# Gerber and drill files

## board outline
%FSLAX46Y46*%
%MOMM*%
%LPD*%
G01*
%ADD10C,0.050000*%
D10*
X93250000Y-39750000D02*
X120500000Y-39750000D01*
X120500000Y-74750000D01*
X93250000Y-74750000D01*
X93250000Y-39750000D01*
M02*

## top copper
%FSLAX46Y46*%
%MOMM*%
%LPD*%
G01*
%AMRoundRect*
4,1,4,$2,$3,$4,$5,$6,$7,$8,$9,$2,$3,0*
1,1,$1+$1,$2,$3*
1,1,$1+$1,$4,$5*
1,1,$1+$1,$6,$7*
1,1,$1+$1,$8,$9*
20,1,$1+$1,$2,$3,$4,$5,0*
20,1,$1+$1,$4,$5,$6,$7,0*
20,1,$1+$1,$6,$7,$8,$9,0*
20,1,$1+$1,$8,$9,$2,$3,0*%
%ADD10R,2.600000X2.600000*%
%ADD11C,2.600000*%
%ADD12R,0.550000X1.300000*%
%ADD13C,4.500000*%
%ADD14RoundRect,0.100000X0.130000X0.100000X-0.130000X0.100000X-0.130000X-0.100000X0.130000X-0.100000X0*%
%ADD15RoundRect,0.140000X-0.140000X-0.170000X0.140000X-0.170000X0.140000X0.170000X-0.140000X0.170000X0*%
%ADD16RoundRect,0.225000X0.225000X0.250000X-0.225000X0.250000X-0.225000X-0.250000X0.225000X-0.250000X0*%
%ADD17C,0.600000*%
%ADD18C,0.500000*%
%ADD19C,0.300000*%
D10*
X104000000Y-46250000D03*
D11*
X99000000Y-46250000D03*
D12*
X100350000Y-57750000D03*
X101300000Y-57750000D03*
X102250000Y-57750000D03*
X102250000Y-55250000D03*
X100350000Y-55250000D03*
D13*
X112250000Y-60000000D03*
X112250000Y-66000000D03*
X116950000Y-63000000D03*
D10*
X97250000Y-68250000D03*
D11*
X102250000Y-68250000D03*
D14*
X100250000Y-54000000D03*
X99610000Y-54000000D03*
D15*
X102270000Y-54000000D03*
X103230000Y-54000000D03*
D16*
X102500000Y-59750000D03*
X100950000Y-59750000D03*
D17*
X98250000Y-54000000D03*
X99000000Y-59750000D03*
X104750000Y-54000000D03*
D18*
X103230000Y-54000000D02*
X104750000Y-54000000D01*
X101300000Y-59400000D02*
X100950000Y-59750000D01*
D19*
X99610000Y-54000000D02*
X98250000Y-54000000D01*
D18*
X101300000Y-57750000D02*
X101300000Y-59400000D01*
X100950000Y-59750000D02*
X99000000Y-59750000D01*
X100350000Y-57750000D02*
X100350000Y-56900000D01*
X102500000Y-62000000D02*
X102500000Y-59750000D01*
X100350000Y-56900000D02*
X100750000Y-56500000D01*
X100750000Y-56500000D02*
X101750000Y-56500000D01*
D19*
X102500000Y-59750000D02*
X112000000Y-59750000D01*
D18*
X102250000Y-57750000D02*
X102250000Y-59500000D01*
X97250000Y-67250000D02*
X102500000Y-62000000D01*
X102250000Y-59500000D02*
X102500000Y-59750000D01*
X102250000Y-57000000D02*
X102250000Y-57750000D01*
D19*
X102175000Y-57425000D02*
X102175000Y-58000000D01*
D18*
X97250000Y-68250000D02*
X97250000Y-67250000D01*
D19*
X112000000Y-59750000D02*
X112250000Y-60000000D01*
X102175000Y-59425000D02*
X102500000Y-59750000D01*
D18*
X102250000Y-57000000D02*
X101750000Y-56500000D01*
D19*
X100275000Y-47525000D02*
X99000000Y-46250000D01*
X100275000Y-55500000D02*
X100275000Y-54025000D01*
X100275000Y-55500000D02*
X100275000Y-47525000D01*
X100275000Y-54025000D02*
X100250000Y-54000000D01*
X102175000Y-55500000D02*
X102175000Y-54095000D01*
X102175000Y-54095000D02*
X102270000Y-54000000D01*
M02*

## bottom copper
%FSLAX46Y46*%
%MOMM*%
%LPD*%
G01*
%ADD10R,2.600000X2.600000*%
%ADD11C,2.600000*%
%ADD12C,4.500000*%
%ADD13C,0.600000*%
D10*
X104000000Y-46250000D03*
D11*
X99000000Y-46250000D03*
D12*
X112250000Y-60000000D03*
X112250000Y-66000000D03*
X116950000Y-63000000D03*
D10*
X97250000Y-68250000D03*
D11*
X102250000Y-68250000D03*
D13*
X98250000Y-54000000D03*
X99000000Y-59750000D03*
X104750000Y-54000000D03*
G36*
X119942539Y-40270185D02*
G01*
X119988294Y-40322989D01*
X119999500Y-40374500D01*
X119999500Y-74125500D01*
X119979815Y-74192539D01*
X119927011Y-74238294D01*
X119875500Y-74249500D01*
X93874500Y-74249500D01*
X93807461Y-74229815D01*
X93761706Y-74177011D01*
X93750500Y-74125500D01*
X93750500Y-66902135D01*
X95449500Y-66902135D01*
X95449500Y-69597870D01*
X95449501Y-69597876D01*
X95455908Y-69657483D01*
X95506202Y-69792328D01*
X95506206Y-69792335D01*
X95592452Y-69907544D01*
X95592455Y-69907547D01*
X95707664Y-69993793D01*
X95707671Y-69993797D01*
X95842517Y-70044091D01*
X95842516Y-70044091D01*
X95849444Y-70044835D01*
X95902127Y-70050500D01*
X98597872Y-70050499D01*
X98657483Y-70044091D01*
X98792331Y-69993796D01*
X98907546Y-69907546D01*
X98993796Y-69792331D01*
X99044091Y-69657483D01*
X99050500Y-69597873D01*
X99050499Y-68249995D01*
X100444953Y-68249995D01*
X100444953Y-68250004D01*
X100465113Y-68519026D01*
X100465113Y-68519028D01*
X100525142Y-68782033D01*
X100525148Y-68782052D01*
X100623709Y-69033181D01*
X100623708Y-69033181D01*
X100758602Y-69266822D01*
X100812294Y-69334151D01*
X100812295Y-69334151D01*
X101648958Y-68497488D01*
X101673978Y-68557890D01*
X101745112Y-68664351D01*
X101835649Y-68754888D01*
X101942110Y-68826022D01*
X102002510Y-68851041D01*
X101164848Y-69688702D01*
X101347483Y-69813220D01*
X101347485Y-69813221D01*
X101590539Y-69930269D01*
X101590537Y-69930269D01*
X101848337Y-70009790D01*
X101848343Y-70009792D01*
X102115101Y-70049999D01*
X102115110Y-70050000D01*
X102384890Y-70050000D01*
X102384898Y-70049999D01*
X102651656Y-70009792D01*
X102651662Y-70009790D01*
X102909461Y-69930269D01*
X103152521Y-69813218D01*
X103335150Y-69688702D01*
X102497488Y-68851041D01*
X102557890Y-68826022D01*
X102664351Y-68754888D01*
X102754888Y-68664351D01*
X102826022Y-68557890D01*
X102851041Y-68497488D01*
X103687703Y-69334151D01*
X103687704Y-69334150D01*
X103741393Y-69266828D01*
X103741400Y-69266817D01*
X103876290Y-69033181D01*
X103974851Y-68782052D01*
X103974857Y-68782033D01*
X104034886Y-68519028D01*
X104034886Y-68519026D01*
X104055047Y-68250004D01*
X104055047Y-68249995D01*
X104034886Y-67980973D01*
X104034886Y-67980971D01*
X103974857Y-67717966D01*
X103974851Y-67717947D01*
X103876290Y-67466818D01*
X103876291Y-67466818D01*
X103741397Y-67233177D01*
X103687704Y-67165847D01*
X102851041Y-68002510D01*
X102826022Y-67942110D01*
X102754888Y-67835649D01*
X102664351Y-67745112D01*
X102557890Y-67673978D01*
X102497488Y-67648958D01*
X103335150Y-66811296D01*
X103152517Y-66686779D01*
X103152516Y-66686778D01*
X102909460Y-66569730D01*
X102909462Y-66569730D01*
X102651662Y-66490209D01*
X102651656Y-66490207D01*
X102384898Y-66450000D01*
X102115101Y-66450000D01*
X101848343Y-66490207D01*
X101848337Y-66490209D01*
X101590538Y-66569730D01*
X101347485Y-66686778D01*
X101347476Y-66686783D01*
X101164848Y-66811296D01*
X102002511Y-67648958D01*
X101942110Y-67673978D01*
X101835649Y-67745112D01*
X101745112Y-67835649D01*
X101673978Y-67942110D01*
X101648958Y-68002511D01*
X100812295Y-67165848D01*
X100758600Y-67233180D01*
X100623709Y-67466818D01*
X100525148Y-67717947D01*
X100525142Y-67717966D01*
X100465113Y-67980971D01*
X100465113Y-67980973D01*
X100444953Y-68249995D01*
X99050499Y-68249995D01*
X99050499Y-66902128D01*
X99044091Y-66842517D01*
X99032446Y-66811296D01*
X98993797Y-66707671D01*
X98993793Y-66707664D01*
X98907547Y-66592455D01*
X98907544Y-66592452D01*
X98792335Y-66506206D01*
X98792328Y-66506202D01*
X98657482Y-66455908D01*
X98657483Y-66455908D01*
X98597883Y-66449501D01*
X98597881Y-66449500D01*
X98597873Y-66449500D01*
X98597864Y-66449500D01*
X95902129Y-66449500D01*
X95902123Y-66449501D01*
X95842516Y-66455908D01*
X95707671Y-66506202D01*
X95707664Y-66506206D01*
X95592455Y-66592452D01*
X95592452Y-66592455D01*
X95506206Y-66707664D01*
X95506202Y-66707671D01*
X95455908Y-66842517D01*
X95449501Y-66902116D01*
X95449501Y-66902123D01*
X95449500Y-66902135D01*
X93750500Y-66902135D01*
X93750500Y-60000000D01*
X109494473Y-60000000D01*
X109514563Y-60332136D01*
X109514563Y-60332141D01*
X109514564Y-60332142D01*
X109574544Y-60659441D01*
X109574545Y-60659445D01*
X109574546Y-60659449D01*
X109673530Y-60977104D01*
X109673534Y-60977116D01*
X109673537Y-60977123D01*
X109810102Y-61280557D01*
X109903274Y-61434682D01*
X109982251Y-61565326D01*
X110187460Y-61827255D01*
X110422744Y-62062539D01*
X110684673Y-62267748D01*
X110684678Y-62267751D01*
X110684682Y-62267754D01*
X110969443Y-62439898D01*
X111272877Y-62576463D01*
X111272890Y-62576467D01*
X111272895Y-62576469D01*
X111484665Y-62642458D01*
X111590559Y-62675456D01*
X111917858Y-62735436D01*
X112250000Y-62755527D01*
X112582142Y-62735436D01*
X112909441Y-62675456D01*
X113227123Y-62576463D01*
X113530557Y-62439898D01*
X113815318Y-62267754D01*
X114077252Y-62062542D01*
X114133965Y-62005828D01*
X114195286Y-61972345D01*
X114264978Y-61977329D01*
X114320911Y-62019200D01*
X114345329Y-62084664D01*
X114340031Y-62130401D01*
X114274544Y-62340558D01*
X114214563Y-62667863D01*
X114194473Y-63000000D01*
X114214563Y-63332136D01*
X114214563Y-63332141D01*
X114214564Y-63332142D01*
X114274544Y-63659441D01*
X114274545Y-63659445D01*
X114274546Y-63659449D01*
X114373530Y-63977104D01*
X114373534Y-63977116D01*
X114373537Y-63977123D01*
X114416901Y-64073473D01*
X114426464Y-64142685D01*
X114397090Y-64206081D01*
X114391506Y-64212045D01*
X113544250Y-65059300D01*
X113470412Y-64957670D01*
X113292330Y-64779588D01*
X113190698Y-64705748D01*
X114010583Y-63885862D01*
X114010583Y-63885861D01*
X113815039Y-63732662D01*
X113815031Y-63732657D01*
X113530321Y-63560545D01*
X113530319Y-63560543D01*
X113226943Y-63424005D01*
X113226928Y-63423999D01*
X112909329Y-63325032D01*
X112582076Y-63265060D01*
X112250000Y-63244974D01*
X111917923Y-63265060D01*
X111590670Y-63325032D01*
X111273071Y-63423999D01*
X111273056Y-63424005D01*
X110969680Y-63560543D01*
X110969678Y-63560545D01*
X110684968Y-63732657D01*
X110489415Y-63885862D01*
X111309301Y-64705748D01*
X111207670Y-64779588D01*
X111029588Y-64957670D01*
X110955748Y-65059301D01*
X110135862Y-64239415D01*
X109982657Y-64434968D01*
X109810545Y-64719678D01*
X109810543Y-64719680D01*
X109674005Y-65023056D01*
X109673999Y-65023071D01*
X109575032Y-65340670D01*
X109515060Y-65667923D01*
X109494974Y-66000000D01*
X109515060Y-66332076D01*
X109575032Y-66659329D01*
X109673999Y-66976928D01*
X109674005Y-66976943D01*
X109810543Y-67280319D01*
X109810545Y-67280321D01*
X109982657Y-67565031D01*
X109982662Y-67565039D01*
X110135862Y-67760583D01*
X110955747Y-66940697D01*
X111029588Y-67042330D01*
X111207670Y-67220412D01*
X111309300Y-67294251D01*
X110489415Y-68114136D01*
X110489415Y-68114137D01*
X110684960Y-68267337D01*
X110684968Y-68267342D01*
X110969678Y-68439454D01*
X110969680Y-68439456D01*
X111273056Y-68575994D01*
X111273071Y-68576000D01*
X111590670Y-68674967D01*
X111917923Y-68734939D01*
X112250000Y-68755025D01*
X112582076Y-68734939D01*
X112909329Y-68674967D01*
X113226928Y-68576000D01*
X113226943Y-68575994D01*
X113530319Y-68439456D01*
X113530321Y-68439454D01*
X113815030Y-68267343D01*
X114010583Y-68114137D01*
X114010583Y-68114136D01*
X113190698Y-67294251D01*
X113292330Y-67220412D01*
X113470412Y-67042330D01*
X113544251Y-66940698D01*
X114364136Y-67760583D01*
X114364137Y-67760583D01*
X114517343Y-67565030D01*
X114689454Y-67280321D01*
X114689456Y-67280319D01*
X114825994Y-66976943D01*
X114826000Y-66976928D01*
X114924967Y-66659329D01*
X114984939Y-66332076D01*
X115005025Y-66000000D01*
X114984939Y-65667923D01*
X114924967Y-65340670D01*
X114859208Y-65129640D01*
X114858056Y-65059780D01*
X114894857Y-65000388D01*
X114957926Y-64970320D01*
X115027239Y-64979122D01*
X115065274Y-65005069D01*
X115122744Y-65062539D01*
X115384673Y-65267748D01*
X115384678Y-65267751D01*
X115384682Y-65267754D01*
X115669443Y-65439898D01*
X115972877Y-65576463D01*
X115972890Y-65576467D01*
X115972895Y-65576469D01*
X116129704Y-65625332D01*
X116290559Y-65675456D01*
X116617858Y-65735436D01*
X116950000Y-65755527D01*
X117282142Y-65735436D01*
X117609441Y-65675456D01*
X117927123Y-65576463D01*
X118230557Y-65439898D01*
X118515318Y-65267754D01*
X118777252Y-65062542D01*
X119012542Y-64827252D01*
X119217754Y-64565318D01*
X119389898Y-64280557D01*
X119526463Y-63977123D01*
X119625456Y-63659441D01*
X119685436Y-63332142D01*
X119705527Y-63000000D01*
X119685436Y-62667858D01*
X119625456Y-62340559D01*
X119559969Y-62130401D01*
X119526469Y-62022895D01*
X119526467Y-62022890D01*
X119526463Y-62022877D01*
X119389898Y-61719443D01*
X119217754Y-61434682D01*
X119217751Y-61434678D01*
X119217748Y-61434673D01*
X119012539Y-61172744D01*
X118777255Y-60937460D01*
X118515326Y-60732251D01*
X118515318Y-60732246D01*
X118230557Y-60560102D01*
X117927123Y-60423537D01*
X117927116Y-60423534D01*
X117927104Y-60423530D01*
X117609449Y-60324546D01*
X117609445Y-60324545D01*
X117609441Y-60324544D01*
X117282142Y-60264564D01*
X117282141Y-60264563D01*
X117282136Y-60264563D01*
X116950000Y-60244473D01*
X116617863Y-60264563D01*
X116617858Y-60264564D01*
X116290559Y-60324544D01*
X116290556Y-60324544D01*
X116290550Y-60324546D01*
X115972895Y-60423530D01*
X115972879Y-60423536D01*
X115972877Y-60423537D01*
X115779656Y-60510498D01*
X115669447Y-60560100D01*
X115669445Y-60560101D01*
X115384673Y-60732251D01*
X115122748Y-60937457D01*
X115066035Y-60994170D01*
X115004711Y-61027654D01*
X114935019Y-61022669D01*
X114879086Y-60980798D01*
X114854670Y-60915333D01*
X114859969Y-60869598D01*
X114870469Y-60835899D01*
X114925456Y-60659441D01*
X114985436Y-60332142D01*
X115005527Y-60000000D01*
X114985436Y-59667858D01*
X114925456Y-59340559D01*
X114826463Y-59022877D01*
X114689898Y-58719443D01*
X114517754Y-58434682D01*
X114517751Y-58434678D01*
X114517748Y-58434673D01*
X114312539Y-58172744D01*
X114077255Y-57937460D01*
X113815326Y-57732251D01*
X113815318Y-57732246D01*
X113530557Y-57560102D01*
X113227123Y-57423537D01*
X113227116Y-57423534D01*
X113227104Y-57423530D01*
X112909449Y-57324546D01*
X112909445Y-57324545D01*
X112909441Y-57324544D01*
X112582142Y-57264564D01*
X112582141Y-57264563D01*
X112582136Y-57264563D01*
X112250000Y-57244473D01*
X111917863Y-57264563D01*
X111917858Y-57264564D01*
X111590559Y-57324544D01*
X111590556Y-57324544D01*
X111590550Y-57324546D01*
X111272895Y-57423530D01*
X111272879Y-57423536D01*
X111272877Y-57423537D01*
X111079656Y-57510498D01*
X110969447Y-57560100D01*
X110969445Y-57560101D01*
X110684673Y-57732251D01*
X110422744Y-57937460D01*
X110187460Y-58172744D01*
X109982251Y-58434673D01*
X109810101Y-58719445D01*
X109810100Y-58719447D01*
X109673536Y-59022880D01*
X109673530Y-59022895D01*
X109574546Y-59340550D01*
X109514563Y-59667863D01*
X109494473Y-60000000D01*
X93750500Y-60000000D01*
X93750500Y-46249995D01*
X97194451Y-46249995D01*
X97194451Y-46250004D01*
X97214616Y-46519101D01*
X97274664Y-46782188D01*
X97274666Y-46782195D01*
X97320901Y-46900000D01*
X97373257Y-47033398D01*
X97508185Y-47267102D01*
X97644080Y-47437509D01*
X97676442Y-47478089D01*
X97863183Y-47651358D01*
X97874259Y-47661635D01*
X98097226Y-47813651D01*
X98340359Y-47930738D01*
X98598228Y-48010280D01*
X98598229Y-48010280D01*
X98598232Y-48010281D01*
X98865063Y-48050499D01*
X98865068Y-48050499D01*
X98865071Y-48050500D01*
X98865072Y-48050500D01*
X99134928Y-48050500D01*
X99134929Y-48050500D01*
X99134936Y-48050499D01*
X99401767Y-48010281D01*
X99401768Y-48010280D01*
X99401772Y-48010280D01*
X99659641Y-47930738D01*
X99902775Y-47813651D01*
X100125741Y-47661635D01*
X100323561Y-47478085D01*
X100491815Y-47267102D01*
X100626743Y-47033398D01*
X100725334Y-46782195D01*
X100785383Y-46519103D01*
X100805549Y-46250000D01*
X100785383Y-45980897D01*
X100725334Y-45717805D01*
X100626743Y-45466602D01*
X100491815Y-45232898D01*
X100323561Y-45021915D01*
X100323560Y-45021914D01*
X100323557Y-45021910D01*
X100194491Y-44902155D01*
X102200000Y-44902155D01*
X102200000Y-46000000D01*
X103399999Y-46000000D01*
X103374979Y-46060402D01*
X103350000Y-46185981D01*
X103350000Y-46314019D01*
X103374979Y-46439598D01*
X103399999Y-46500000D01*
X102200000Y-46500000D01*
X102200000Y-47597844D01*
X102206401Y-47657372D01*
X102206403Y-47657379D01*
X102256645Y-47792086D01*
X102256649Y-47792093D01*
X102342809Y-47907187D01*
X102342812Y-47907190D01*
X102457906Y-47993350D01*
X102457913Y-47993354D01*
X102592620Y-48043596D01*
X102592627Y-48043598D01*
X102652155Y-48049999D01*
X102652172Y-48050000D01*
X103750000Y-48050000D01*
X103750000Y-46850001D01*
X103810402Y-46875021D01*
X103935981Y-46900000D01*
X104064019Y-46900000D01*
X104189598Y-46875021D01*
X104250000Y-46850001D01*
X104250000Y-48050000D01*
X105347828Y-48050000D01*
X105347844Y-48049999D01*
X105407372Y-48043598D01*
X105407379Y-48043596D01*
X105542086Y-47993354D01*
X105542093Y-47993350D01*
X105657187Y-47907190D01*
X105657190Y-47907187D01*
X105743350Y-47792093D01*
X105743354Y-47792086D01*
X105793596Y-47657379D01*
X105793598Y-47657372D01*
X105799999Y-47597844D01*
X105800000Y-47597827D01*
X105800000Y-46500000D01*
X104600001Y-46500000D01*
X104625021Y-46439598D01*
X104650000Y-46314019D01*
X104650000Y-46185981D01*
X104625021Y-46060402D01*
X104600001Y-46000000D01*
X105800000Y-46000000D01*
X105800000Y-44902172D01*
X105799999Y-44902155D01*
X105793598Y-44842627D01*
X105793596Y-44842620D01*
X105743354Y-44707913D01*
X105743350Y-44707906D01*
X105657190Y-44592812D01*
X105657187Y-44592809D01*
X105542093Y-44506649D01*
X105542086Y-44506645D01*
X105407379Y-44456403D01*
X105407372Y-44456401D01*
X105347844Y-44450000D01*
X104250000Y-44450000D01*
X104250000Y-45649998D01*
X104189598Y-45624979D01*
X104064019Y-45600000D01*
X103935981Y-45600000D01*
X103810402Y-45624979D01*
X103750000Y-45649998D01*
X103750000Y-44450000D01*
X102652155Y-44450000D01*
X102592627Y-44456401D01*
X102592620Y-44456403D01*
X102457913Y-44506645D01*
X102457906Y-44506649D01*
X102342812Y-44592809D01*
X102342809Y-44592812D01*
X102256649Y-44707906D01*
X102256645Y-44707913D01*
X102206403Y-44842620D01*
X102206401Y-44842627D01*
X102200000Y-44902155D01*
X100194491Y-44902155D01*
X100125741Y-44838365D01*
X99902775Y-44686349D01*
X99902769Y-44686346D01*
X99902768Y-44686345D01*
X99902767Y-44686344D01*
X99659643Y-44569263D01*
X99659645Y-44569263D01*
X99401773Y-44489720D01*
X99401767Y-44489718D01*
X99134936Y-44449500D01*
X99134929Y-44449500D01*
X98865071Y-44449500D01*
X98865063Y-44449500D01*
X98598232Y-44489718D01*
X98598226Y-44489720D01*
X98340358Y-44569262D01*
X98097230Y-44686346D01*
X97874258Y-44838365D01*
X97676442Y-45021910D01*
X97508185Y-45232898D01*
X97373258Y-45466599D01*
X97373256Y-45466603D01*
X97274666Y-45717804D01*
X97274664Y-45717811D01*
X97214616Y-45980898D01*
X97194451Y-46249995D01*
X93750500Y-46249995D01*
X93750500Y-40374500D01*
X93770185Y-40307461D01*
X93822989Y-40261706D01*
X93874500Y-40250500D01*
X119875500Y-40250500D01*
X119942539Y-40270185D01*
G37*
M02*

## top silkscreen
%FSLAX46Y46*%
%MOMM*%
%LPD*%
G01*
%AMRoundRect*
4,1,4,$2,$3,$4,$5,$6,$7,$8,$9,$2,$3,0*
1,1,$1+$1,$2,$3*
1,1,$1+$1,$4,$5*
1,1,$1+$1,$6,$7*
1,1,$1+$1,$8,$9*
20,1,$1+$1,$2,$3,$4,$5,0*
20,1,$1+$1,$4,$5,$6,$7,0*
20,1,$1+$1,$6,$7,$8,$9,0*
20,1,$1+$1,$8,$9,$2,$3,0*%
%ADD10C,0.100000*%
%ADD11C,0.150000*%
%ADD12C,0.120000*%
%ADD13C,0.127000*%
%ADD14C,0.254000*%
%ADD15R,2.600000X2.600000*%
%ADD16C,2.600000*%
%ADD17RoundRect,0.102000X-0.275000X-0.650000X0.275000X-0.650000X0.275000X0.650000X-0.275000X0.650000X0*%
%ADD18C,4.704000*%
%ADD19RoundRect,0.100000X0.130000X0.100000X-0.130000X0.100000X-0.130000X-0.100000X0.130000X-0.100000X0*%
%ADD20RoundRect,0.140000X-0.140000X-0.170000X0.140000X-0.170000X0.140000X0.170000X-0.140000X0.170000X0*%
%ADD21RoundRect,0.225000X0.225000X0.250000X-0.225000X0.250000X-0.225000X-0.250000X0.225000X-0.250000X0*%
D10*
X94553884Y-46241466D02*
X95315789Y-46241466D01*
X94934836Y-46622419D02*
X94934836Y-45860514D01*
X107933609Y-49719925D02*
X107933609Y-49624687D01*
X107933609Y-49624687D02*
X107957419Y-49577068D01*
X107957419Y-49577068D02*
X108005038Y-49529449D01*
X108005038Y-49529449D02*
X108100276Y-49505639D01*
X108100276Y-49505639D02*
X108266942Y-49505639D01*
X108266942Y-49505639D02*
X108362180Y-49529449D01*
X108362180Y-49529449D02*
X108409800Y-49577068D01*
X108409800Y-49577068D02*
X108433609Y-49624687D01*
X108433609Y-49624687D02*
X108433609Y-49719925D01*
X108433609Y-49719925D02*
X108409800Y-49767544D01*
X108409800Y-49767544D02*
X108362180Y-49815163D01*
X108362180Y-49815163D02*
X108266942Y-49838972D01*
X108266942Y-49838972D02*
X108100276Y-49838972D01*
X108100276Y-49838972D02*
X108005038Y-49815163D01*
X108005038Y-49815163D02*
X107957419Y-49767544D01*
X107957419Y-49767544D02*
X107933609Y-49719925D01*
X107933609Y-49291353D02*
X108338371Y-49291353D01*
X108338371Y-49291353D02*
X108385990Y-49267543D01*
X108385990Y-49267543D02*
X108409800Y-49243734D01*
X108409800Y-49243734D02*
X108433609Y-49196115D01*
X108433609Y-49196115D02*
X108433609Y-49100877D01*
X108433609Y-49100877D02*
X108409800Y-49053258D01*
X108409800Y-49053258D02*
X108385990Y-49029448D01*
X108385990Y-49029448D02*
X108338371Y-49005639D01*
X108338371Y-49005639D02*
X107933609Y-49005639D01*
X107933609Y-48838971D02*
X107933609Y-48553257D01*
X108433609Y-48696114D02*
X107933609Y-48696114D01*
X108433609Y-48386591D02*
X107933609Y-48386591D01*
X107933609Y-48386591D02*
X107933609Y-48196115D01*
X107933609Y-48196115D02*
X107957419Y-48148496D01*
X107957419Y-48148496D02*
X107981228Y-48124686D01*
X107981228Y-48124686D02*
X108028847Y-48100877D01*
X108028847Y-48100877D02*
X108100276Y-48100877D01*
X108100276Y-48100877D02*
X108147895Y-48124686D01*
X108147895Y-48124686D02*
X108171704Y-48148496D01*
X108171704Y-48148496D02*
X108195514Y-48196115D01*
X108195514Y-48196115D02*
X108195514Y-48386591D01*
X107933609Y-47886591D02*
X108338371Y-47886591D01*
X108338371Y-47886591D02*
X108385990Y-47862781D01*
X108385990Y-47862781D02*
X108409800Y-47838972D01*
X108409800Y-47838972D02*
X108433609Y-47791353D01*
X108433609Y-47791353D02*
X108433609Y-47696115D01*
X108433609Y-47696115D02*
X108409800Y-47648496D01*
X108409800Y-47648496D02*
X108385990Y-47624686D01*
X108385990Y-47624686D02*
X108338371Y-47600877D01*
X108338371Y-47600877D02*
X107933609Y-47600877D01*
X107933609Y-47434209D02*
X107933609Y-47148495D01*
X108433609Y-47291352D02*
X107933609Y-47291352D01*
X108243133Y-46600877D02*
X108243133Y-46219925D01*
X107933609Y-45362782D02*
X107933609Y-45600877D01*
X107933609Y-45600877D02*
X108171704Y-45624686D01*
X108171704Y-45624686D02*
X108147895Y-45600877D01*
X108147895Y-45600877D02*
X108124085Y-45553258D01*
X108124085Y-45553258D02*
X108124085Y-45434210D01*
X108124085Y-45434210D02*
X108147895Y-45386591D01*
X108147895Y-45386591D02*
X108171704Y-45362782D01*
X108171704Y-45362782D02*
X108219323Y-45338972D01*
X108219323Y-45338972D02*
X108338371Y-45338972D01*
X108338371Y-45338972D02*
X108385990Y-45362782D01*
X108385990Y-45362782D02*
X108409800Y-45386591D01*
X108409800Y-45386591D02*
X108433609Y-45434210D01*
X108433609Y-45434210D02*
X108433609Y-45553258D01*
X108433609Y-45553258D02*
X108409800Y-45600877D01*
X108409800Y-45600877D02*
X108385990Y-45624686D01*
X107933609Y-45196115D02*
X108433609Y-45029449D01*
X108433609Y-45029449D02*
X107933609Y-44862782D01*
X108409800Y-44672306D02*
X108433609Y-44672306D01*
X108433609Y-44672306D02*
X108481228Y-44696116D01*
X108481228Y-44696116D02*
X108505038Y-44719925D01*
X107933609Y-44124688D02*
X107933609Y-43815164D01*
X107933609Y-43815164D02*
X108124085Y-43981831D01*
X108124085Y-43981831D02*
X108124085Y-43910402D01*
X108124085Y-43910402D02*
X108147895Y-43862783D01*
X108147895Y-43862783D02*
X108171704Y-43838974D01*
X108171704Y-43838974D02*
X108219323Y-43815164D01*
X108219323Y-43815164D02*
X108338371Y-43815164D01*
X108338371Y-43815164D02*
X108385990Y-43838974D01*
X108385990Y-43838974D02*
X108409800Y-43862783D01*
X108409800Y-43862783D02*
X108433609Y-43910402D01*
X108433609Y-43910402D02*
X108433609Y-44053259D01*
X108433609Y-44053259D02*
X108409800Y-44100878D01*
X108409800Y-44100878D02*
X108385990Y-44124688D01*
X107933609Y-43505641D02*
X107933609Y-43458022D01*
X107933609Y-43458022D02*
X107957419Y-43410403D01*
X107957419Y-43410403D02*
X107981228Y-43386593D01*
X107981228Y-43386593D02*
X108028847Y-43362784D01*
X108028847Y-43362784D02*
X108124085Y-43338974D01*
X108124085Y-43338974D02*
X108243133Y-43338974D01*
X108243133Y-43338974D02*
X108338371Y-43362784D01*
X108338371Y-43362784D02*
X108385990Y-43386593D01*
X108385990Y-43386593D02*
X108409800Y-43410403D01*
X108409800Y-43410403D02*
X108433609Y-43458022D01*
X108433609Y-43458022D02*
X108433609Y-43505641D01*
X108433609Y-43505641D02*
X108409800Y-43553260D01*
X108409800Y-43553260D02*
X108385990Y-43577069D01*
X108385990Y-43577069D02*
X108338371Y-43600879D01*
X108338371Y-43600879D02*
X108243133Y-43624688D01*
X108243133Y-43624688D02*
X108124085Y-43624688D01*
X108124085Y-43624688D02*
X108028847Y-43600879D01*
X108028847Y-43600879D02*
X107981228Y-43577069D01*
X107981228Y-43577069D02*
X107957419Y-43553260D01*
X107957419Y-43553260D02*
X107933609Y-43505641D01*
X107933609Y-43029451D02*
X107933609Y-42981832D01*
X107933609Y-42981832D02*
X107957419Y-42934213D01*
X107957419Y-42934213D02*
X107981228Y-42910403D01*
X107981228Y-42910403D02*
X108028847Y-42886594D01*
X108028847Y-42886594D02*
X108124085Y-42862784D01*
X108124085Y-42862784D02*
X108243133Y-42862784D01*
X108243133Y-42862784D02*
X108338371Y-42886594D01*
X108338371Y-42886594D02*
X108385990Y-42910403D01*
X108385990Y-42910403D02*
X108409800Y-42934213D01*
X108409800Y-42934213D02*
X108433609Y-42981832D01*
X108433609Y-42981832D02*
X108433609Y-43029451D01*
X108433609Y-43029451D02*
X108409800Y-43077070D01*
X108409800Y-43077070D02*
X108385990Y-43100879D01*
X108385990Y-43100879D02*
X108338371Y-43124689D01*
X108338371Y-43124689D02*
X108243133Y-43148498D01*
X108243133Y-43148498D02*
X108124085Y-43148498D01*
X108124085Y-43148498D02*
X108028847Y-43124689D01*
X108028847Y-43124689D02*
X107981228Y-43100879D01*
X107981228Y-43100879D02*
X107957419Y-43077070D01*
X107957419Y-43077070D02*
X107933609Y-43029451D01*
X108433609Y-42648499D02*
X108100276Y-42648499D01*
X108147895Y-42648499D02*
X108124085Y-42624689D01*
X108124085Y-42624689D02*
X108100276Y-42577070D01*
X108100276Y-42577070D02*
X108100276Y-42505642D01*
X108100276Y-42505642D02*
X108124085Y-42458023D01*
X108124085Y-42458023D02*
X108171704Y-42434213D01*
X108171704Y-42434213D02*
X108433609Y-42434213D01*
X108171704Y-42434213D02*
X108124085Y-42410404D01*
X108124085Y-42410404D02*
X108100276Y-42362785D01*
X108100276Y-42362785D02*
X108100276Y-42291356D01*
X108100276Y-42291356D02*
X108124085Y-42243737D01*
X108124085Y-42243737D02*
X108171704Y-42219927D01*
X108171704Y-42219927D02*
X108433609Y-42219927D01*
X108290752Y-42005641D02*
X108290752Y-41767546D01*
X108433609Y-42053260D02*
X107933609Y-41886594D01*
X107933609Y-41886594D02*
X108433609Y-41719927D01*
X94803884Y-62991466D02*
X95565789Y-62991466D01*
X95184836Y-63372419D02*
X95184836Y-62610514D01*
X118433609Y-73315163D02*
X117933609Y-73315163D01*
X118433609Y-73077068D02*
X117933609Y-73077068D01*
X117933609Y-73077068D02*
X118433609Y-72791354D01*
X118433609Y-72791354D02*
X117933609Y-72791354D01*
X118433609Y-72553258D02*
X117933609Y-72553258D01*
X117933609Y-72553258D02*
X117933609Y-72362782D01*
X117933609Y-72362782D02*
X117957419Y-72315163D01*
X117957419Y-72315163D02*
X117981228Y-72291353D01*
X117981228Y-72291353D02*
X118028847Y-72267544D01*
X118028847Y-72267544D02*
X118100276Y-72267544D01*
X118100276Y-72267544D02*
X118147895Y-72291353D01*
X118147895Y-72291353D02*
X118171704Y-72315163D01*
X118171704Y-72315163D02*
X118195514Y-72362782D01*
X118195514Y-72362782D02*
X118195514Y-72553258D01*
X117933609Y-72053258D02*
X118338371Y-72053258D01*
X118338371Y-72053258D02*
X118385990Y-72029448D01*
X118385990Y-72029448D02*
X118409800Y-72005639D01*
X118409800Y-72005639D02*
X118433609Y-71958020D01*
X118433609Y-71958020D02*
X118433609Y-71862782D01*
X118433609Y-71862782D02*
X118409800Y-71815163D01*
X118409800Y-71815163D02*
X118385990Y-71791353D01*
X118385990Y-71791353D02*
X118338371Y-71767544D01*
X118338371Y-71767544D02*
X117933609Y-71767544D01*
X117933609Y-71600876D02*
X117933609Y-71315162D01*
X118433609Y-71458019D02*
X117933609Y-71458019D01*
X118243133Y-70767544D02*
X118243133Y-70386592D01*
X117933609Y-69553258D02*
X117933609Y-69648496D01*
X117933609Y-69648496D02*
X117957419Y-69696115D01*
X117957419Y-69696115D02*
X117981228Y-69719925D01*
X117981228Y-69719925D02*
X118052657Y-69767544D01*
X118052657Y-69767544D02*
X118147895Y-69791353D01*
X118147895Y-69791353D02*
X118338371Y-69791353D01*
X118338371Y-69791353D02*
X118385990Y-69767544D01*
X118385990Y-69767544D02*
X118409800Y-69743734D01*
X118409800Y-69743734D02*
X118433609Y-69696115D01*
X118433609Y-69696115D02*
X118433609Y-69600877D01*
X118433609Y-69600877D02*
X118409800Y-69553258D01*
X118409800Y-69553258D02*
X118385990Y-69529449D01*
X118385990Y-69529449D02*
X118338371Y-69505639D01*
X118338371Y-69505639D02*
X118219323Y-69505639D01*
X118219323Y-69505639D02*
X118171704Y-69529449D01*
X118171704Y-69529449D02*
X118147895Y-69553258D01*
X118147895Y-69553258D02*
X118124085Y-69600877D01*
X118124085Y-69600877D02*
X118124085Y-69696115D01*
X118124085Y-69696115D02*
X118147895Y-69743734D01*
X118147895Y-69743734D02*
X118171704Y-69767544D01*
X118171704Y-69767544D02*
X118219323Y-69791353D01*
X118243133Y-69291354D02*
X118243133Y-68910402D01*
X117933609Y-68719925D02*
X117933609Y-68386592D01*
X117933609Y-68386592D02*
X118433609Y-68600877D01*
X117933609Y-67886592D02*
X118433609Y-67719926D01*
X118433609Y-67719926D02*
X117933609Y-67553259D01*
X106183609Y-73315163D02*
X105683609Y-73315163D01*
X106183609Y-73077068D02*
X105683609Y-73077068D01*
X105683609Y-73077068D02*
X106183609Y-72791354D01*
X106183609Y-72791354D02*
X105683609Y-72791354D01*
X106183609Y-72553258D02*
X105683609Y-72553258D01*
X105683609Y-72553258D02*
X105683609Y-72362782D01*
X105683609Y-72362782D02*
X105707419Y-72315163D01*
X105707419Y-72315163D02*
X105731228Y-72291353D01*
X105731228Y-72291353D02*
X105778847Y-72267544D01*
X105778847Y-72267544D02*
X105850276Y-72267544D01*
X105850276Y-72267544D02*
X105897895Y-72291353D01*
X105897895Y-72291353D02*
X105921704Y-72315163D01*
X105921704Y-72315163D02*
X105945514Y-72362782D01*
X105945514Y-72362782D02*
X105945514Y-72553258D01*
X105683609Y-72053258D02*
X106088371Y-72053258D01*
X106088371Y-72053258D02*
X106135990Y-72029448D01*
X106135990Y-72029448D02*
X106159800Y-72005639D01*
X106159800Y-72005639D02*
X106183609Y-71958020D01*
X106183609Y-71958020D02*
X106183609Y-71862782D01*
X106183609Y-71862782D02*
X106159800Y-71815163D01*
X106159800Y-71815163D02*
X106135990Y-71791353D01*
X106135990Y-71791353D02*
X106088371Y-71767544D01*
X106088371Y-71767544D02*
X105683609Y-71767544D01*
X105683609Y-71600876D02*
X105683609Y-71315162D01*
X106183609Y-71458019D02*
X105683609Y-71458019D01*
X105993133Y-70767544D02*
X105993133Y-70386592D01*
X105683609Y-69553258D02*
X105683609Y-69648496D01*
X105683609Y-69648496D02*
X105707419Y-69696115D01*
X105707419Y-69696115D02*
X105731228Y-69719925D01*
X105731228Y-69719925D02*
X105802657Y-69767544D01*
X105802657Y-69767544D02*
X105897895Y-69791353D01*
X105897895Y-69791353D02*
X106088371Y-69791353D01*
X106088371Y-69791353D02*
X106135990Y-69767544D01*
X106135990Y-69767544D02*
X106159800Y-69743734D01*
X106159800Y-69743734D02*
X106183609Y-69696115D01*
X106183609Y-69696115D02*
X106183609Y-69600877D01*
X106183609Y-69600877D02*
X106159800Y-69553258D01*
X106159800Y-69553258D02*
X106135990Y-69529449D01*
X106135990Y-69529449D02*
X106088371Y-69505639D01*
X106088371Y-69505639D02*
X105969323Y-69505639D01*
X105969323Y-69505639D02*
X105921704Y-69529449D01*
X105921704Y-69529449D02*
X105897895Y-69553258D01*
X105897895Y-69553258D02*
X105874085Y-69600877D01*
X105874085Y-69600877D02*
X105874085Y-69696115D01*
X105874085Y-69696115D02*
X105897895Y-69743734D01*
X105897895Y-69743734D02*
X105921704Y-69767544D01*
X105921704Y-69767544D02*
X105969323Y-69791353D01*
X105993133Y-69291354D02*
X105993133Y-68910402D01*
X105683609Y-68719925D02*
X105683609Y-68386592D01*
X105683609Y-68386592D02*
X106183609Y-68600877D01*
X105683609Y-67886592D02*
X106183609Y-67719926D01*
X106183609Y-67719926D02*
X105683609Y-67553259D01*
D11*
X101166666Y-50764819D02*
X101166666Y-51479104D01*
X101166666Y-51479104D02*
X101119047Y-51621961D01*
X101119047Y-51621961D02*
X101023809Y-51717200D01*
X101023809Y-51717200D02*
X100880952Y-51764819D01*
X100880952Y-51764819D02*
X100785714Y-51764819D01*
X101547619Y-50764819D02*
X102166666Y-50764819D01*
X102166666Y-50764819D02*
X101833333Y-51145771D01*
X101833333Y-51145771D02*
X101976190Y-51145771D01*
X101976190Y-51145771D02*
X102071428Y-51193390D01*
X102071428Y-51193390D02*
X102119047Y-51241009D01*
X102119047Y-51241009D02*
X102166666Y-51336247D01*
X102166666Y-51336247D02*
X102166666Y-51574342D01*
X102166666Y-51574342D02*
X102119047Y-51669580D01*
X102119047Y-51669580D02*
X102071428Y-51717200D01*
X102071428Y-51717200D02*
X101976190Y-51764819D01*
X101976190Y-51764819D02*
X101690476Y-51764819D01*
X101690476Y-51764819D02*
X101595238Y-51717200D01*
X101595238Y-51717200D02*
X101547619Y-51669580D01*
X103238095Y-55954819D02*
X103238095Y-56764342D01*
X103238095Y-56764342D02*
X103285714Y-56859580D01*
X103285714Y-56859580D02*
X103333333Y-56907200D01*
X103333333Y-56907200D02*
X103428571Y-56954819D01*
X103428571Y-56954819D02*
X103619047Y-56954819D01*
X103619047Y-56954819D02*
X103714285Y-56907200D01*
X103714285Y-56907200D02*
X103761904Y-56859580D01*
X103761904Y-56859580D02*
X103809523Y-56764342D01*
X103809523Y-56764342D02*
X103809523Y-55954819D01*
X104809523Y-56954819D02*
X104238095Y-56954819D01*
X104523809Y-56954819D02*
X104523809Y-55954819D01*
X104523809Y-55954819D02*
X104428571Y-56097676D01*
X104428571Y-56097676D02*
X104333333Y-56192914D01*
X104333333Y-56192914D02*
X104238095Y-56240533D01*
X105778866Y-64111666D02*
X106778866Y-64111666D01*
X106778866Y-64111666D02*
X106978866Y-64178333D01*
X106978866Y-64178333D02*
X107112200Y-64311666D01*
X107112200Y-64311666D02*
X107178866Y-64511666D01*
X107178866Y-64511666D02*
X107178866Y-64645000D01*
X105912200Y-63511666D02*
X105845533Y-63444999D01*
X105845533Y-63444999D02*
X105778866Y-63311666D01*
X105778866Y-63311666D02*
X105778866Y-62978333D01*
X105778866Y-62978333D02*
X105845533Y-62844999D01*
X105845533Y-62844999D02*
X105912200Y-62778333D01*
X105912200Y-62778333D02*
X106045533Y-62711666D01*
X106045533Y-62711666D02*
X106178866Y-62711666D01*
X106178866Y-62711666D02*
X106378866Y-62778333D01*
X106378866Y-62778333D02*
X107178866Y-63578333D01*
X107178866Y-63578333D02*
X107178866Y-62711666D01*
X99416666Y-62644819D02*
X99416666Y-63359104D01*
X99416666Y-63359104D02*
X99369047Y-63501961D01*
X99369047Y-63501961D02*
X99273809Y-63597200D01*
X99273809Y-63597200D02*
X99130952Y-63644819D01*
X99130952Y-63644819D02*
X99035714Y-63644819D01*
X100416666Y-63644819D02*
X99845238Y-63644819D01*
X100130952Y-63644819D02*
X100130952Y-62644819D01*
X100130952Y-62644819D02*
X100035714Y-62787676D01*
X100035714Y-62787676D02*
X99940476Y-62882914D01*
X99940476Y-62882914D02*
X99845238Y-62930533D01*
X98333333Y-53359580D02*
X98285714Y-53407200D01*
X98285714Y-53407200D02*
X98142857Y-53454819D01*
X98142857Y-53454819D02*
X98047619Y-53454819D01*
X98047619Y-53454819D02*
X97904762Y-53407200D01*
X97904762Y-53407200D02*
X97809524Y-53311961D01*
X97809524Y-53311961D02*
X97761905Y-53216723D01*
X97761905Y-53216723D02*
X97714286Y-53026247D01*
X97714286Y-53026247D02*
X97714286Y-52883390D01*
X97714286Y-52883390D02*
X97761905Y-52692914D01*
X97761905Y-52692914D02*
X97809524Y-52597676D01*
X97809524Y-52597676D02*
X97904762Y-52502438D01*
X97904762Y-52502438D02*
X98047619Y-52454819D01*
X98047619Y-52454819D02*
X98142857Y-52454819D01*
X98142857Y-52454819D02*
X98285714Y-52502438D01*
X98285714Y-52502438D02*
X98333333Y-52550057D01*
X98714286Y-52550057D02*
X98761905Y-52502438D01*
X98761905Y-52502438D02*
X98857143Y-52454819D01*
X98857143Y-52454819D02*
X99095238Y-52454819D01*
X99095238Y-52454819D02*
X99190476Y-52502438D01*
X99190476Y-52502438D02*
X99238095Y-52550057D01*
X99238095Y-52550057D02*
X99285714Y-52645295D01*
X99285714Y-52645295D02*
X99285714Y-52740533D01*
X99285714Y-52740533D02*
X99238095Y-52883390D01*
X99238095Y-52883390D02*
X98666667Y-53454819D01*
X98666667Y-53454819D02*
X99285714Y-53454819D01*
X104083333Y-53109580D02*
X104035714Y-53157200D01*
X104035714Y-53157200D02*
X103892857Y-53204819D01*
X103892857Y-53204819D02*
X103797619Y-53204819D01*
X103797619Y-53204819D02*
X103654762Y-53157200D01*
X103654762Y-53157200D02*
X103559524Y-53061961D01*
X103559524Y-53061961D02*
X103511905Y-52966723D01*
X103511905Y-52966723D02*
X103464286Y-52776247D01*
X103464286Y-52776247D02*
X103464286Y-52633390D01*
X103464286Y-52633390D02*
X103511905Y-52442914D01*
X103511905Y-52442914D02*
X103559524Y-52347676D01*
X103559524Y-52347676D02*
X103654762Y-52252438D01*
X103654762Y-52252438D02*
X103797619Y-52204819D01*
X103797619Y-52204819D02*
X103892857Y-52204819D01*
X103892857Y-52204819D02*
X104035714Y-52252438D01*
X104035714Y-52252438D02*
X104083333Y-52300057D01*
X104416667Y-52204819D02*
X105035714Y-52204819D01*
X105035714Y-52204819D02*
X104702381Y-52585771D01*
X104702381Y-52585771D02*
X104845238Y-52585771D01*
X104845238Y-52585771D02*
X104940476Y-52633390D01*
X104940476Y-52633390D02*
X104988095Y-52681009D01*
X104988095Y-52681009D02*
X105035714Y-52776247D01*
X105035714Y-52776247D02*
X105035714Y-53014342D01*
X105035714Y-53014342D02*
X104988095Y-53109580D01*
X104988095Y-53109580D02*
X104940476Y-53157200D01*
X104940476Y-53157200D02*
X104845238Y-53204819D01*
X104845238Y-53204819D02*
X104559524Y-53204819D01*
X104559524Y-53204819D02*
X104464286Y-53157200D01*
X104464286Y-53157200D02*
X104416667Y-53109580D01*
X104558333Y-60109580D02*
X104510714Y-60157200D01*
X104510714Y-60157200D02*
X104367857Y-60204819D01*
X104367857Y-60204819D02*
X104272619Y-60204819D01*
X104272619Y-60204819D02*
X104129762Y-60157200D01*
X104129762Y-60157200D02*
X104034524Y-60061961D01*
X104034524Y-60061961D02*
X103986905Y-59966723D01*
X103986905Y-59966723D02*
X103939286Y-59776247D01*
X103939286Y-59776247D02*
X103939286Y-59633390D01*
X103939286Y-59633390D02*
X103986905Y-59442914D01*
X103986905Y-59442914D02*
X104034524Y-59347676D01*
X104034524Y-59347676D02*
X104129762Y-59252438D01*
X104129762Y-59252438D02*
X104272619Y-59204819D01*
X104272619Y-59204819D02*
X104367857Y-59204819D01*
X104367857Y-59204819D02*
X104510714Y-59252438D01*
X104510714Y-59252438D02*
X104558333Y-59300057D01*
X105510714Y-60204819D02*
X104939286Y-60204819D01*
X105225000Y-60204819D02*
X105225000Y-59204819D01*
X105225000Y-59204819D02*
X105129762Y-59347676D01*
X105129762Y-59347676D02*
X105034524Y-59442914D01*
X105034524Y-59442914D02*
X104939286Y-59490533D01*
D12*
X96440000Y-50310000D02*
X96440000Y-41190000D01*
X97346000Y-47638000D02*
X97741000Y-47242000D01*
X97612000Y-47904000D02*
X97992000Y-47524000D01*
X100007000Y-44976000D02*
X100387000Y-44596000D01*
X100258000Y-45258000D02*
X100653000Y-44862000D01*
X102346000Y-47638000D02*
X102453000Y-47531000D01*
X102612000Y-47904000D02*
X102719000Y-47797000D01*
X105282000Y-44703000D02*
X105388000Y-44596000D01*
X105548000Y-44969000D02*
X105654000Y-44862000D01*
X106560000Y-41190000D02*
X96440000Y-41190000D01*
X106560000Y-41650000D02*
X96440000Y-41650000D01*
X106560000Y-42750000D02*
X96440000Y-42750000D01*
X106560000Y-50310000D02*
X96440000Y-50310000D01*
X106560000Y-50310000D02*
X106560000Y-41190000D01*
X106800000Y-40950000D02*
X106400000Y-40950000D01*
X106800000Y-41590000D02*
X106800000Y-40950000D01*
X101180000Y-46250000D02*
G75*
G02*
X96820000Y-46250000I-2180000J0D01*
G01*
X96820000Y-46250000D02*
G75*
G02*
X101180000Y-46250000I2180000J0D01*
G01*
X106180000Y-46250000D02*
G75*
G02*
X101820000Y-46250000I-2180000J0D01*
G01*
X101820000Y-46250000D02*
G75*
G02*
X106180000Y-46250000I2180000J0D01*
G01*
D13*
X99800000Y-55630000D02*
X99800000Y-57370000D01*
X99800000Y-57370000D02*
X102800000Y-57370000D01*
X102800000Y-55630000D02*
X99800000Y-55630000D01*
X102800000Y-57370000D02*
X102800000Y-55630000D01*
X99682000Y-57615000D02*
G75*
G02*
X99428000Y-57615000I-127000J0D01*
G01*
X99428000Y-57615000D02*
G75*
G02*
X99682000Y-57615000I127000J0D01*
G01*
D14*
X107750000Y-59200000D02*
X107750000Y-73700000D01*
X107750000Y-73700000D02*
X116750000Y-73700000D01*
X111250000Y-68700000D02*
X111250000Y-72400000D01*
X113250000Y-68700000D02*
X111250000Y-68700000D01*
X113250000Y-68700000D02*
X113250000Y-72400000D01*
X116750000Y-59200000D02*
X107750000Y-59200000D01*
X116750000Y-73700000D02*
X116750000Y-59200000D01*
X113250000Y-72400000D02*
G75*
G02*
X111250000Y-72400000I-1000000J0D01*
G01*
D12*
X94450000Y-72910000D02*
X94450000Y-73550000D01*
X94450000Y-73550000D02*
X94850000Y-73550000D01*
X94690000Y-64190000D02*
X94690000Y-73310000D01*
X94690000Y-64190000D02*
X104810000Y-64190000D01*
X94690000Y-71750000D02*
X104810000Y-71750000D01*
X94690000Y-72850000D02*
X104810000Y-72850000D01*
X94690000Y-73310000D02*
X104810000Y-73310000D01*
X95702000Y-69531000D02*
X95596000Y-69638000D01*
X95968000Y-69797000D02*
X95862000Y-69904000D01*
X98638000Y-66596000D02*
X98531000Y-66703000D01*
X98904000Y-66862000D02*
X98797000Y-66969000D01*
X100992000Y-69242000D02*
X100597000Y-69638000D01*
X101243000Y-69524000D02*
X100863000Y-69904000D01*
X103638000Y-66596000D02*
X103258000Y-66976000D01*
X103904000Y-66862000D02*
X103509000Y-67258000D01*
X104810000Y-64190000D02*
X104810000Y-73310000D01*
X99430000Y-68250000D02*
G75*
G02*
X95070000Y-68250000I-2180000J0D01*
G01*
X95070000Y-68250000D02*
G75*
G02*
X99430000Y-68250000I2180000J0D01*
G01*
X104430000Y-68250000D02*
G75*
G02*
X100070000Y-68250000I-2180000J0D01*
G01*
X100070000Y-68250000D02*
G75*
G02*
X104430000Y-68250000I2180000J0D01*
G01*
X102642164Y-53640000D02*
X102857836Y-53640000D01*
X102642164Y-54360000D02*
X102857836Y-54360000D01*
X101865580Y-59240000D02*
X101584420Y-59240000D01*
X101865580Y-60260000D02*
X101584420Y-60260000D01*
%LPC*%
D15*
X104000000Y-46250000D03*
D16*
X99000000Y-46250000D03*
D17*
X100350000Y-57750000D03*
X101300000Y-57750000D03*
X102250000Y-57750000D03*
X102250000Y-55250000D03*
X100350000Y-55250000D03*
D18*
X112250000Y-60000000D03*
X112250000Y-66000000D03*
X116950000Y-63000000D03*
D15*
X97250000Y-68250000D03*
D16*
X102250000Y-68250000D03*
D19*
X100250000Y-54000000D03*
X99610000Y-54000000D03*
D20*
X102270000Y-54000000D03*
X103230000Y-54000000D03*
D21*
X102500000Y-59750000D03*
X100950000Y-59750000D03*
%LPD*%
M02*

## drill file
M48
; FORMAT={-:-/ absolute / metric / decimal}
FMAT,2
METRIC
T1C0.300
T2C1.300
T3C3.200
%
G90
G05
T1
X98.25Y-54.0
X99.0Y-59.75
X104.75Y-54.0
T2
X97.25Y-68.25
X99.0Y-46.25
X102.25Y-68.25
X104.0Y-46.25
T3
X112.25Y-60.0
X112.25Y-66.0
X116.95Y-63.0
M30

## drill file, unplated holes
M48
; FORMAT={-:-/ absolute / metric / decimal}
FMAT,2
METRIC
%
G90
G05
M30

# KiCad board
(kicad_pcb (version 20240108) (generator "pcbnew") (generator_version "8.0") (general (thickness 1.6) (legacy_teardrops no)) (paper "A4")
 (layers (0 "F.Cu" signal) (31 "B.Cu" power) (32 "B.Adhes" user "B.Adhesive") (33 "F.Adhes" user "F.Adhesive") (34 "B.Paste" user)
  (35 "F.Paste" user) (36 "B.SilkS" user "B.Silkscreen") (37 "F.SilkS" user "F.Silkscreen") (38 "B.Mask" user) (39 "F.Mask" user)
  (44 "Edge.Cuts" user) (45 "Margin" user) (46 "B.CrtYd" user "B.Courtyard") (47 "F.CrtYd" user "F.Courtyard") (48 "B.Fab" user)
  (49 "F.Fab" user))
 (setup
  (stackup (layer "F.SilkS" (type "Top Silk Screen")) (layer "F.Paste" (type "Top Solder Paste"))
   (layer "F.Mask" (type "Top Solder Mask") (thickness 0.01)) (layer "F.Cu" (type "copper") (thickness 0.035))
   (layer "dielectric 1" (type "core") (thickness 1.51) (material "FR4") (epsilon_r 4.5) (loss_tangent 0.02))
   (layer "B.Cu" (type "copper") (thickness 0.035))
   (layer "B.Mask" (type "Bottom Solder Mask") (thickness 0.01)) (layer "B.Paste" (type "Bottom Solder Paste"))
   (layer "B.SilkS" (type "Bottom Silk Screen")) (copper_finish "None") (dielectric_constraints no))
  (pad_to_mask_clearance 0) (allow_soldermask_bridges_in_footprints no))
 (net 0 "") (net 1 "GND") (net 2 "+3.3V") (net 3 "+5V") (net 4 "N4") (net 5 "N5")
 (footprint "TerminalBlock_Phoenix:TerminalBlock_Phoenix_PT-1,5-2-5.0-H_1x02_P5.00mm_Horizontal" (layer "F.Cu") (at 104 46.25 180)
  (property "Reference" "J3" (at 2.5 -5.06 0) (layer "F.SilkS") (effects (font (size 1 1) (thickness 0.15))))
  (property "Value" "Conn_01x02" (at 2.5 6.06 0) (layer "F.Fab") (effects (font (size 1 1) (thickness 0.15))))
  (fp_line (start 7.56 -4.06) (end 7.56 5.06) (stroke (width 0.12) (type solid)) (layer "F.SilkS"))
  (fp_line (start 6.654 -1.388) (end 6.259 -0.992) (stroke (width 0.12) (type solid)) (layer "F.SilkS"))
  (fp_line (start 6.388 -1.654) (end 6.008 -1.274) (stroke (width 0.12) (type solid)) (layer "F.SilkS"))
  (fp_line (start 3.993 1.274) (end 3.613 1.654) (stroke (width 0.12) (type solid)) (layer "F.SilkS"))
  (fp_line (start 3.742 0.992) (end 3.347 1.388) (stroke (width 0.12) (type solid)) (layer "F.SilkS"))
  (fp_line (start 1.654 -1.388) (end 1.547 -1.281) (stroke (width 0.12) (type solid)) (layer "F.SilkS"))
  (fp_line (start 1.388 -1.654) (end 1.281 -1.547) (stroke (width 0.12) (type solid)) (layer "F.SilkS"))
  (fp_line (start -1.282 1.547) (end -1.388 1.654) (stroke (width 0.12) (type solid)) (layer "F.SilkS"))
  (fp_line (start -1.548 1.281) (end -1.654 1.388) (stroke (width 0.12) (type solid)) (layer "F.SilkS"))
  (fp_line (start -2.56 5.06) (end 7.56 5.06) (stroke (width 0.12) (type solid)) (layer "F.SilkS"))
  (fp_line (start -2.56 4.6) (end 7.56 4.6) (stroke (width 0.12) (type solid)) (layer "F.SilkS"))
  (fp_line (start -2.56 3.5) (end 7.56 3.5) (stroke (width 0.12) (type solid)) (layer "F.SilkS"))
  (fp_line (start -2.56 -4.06) (end 7.56 -4.06) (stroke (width 0.12) (type solid)) (layer "F.SilkS"))
  (fp_line (start -2.56 -4.06) (end -2.56 5.06) (stroke (width 0.12) (type solid)) (layer "F.SilkS"))
  (fp_line (start -2.8 5.3) (end -2.4 5.3) (stroke (width 0.12) (type solid)) (layer "F.SilkS"))
  (fp_line (start -2.8 4.66) (end -2.8 5.3) (stroke (width 0.12) (type solid)) (layer "F.SilkS"))
  (fp_circle (center 5 0) (end 7.18 0) (stroke (width 0.12) (type solid)) (fill none) (layer "F.SilkS"))
  (fp_circle (center 0 0) (end 2.18 0) (stroke (width 0.12) (type solid)) (fill none) (layer "F.SilkS"))
  (pad "1" thru_hole rect (at 0 0 180) (size 2.6 2.6) (drill 1.3) (layers "*.Cu" "*.Mask") (remove_unused_layers no) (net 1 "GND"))
  (pad "2" thru_hole circle (at 5 0 180) (size 2.6 2.6) (drill 1.3) (layers "*.Cu" "*.Mask") (remove_unused_layers no) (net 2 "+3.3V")))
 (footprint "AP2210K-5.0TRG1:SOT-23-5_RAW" (layer "F.Cu") (at 101.3 56.5)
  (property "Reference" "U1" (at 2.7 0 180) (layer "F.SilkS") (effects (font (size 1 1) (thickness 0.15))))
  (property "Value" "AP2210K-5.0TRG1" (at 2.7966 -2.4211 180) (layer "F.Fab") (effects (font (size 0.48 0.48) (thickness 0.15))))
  (fp_line (start -1.5 -0.87) (end -1.5 0.87) (stroke (width 0.127) (type solid)) (layer "F.SilkS"))
  (fp_line (start -1.5 0.87) (end 1.5 0.87) (stroke (width 0.127) (type solid)) (layer "F.SilkS"))
  (fp_line (start 1.5 -0.87) (end -1.5 -0.87) (stroke (width 0.127) (type solid)) (layer "F.SilkS"))
  (fp_line (start 1.5 0.87) (end 1.5 -0.87) (stroke (width 0.127) (type solid)) (layer "F.SilkS"))
  (fp_circle (center -1.745 1.115) (end -1.618 1.115) (stroke (width 0.127) (type solid)) (fill none) (layer "F.SilkS"))
  (pad "1" smd rect (at -0.95 1.25) (size 0.55 1.3) (layers "F.Cu" "F.Paste" "F.Mask") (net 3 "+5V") (solder_mask_margin 0.102))
  (pad "2" smd rect (at 0 1.25) (size 0.55 1.3) (layers "F.Cu" "F.Paste" "F.Mask") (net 1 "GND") (solder_mask_margin 0.102))
  (pad "3" smd rect (at 0.95 1.25) (size 0.55 1.3) (layers "F.Cu" "F.Paste" "F.Mask") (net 3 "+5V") (solder_mask_margin 0.102))
  (pad "4" smd rect (at 0.95 -1.25) (size 0.55 1.3) (layers "F.Cu" "F.Paste" "F.Mask") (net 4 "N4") (solder_mask_margin 0.102))
  (pad "5" smd rect (at -0.95 -1.25) (size 0.55 1.3) (layers "F.Cu" "F.Paste" "F.Mask") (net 2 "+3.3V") (solder_mask_margin 0.102)))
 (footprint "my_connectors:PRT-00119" (layer "F.Cu") (at 112.25 73.7 -90)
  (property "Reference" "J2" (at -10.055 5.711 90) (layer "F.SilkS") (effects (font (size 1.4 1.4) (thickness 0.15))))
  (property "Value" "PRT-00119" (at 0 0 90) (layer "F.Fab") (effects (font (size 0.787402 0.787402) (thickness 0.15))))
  (fp_line (start -14.5 4.5) (end 0 4.5) (stroke (width 0.254) (type solid)) (layer "F.SilkS"))
  (fp_line (start 0 4.5) (end 0 -4.5) (stroke (width 0.254) (type solid)) (layer "F.SilkS"))
  (fp_line (start -5 1) (end -1.3 1) (stroke (width 0.254) (type solid)) (layer "F.SilkS"))
  (fp_line (start -5 -1) (end -5 1) (stroke (width 0.254) (type solid)) (layer "F.SilkS"))
  (fp_line (start -5 -1) (end -1.3 -1) (stroke (width 0.254) (type solid)) (layer "F.SilkS"))
  (fp_line (start -14.5 -4.5) (end -14.5 4.5) (stroke (width 0.254) (type solid)) (layer "F.SilkS"))
  (fp_line (start 0 -4.5) (end -14.5 -4.5) (stroke (width 0.254) (type solid)) (layer "F.SilkS"))
  (fp_arc (start -1.3 -1) (mid -0.3 0) (end -1.3 1) (stroke (width 0.254) (type solid)) (layer "F.SilkS"))
  (pad "1" thru_hole circle (at -13.7 0 270) (size 4.5 4.5) (drill 3.2) (layers "*.Cu" "*.Mask") (remove_unused_layers no) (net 3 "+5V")
   (solder_mask_margin 0.102))
  (pad "2" thru_hole circle (at -7.7 0 270) (size 4.5 4.5) (drill 3.2) (layers "*.Cu" "*.Mask") (remove_unused_layers no) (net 1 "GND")
   (solder_mask_margin 0.102))
  (pad "3" thru_hole circle (at -10.7 -4.7 270) (size 4.5 4.5) (drill 3.2) (layers "*.Cu" "*.Mask") (remove_unused_layers no) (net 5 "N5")
   (solder_mask_margin 0.102)))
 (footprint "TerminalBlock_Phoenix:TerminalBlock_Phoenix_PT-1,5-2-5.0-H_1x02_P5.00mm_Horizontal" (layer "F.Cu") (at 97.25 68.25)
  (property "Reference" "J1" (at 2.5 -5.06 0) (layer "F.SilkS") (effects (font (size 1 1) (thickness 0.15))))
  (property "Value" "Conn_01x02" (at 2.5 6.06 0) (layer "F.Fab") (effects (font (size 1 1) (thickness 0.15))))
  (fp_line (start -2.8 4.66) (end -2.8 5.3) (stroke (width 0.12) (type solid)) (layer "F.SilkS"))
  (fp_line (start -2.8 5.3) (end -2.4 5.3) (stroke (width 0.12) (type solid)) (layer "F.SilkS"))
  (fp_line (start -2.56 -4.06) (end -2.56 5.06) (stroke (width 0.12) (type solid)) (layer "F.SilkS"))
  (fp_line (start -2.56 -4.06) (end 7.56 -4.06) (stroke (width 0.12) (type solid)) (layer "F.SilkS"))
  (fp_line (start -2.56 3.5) (end 7.56 3.5) (stroke (width 0.12) (type solid)) (layer "F.SilkS"))
  (fp_line (start -2.56 4.6) (end 7.56 4.6) (stroke (width 0.12) (type solid)) (layer "F.SilkS"))
  (fp_line (start -2.56 5.06) (end 7.56 5.06) (stroke (width 0.12) (type solid)) (layer "F.SilkS"))
  (fp_line (start -1.548 1.281) (end -1.654 1.388) (stroke (width 0.12) (type solid)) (layer "F.SilkS"))
  (fp_line (start -1.282 1.547) (end -1.388 1.654) (stroke (width 0.12) (type solid)) (layer "F.SilkS"))
  (fp_line (start 1.388 -1.654) (end 1.281 -1.547) (stroke (width 0.12) (type solid)) (layer "F.SilkS"))
  (fp_line (start 1.654 -1.388) (end 1.547 -1.281) (stroke (width 0.12) (type solid)) (layer "F.SilkS"))
  (fp_line (start 3.742 0.992) (end 3.347 1.388) (stroke (width 0.12) (type solid)) (layer "F.SilkS"))
  (fp_line (start 3.993 1.274) (end 3.613 1.654) (stroke (width 0.12) (type solid)) (layer "F.SilkS"))
  (fp_line (start 6.388 -1.654) (end 6.008 -1.274) (stroke (width 0.12) (type solid)) (layer "F.SilkS"))
  (fp_line (start 6.654 -1.388) (end 6.259 -0.992) (stroke (width 0.12) (type solid)) (layer "F.SilkS"))
  (fp_line (start 7.56 -4.06) (end 7.56 5.06) (stroke (width 0.12) (type solid)) (layer "F.SilkS"))
  (fp_circle (center 0 0) (end 2.18 0) (stroke (width 0.12) (type solid)) (fill none) (layer "F.SilkS"))
  (fp_circle (center 5 0) (end 7.18 0) (stroke (width 0.12) (type solid)) (fill none) (layer "F.SilkS"))
  (pad "1" thru_hole rect (at 0 0) (size 2.6 2.6) (drill 1.3) (layers "*.Cu" "*.Mask") (remove_unused_layers no) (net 3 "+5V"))
  (pad "2" thru_hole circle (at 5 0) (size 2.6 2.6) (drill 1.3) (layers "*.Cu" "*.Mask") (remove_unused_layers no) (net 1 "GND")))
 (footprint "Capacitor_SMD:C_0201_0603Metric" (layer "F.Cu") (at 99.93 54 180)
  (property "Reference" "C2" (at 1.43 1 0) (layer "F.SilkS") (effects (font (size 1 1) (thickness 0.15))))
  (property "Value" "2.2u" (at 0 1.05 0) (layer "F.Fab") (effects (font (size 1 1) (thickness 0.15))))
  (pad "" smd roundrect (at -0.345 0 180) (size 0.318 0.36) (layers "F.Paste") (roundrect_rratio 0.25))
  (pad "" smd roundrect (at 0.345 0 180) (size 0.318 0.36) (layers "F.Paste") (roundrect_rratio 0.25))
  (pad "1" smd roundrect (at -0.32 0 180) (size 0.46 0.4) (layers "F.Cu" "F.Mask") (roundrect_rratio 0.25) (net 2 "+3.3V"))
  (pad "2" smd roundrect (at 0.32 0 180) (size 0.46 0.4) (layers "F.Cu" "F.Mask") (roundrect_rratio 0.25) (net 1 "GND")))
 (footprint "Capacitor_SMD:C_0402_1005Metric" (layer "F.Cu") (at 102.75 54)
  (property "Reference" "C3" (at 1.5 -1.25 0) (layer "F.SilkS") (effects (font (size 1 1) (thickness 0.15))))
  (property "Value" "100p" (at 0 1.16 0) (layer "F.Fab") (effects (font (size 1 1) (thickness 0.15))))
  (fp_line (start -0.107836 -0.36) (end 0.107836 -0.36) (stroke (width 0.12) (type solid)) (layer "F.SilkS"))
  (fp_line (start -0.107836 0.36) (end 0.107836 0.36) (stroke (width 0.12) (type solid)) (layer "F.SilkS"))
  (pad "1" smd roundrect (at -0.48 0) (size 0.56 0.62) (layers "F.Cu" "F.Paste" "F.Mask") (roundrect_rratio 0.25) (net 4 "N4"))
  (pad "2" smd roundrect (at 0.48 0) (size 0.56 0.62) (layers "F.Cu" "F.Paste" "F.Mask") (roundrect_rratio 0.25) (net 1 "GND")))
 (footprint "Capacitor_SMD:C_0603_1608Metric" (layer "F.Cu") (at 101.725 59.75 180)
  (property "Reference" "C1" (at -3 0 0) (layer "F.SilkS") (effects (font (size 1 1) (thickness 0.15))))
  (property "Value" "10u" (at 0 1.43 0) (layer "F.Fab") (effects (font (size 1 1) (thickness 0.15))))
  (fp_line (start -0.14058 0.51) (end 0.14058 0.51) (stroke (width 0.12) (type solid)) (layer "F.SilkS"))
  (fp_line (start -0.14058 -0.51) (end 0.14058 -0.51) (stroke (width 0.12) (type solid)) (layer "F.SilkS"))
  (pad "1" smd roundrect (at -0.775 0 180) (size 0.9 0.95) (layers "F.Cu" "F.Paste" "F.Mask") (roundrect_rratio 0.25) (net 3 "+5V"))
  (pad "2" smd roundrect (at 0.775 0 180) (size 0.9 0.95) (layers "F.Cu" "F.Paste" "F.Mask") (roundrect_rratio 0.25) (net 1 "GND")))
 (gr_rect (start 93.25 39.75) (end 120.5 74.75) (stroke (width 0.05) (type default)) (fill none) (layer "Edge.Cuts"))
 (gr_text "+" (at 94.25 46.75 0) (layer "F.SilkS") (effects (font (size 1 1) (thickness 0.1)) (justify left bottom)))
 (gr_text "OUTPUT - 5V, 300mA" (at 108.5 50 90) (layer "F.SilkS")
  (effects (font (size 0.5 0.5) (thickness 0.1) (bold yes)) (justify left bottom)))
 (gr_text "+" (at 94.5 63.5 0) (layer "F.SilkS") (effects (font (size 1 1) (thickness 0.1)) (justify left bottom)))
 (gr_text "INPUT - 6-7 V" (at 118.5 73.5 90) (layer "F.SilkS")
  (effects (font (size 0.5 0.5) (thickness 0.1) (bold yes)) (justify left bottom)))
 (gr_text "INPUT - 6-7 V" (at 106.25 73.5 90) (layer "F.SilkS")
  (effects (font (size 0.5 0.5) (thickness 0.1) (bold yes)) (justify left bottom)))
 (segment (start 103.23 54) (end 104.75 54) (width 0.5) (layer "F.Cu") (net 1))
 (segment (start 101.3 59.4) (end 100.95 59.75) (width 0.5) (layer "F.Cu") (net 1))
 (segment (start 99.61 54) (end 98.25 54) (width 0.3) (layer "F.Cu") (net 1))
 (segment (start 101.3 57.75) (end 101.3 59.4) (width 0.5) (layer "F.Cu") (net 1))
 (segment (start 100.95 59.75) (end 99 59.75) (width 0.5) (layer "F.Cu") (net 1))
 (via (at 98.25 54) (size 0.6) (drill 0.3) (layers "F.Cu" "B.Cu") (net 1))
 (via (at 99 59.75) (size 0.6) (drill 0.3) (layers "F.Cu" "B.Cu") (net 1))
 (via (at 104.75 54) (size 0.6) (drill 0.3) (layers "F.Cu" "B.Cu") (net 1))
 (segment (start 100.35 57.75) (end 100.35 56.9) (width 0.5) (layer "F.Cu") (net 3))
 (segment (start 102.5 62) (end 102.5 59.75) (width 0.5) (layer "F.Cu") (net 3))
 (segment (start 100.35 56.9) (end 100.75 56.5) (width 0.5) (layer "F.Cu") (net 3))
 (segment (start 100.75 56.5) (end 101.75 56.5) (width 0.5) (layer "F.Cu") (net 3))
 (segment (start 102.5 59.75) (end 112 59.75) (width 0.3) (layer "F.Cu") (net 3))
 (segment (start 102.25 57.75) (end 102.25 59.5) (width 0.5) (layer "F.Cu") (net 3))
 (segment (start 97.25 67.25) (end 102.5 62) (width 0.5) (layer "F.Cu") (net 3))
 (segment (start 102.25 59.5) (end 102.5 59.75) (width 0.5) (layer "F.Cu") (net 3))
 (segment (start 102.25 57) (end 102.25 57.75) (width 0.5) (layer "F.Cu") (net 3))
 (segment (start 102.175 57.425) (end 102.175 58) (width 0.3) (layer "F.Cu") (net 3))
 (segment (start 97.25 68.25) (end 97.25 67.25) (width 0.5) (layer "F.Cu") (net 3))
 (segment (start 112 59.75) (end 112.25 60) (width 0.3) (layer "F.Cu") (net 3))
 (segment (start 102.175 59.425) (end 102.5 59.75) (width 0.3) (layer "F.Cu") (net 3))
 (segment (start 102.25 57) (end 101.75 56.5) (width 0.5) (layer "F.Cu") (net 3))
 (segment (start 100.275 47.525) (end 99 46.25) (width 0.3) (layer "F.Cu") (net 2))
 (segment (start 100.275 55.5) (end 100.275 54.025) (width 0.3) (layer "F.Cu") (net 2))
 (segment (start 100.275 55.5) (end 100.275 47.525) (width 0.3) (layer "F.Cu") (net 2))
 (segment (start 100.275 54.025) (end 100.25 54) (width 0.3) (layer "F.Cu") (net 2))
 (segment (start 102.175 55.5) (end 102.175 54.095) (width 0.3) (layer "F.Cu") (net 4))
 (segment (start 102.175 54.095) (end 102.27 54) (width 0.3) (layer "F.Cu") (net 4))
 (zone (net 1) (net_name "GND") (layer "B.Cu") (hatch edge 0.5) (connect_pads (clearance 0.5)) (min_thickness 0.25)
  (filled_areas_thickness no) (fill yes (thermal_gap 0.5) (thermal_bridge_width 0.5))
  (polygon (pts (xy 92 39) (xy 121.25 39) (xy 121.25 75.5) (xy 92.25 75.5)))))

